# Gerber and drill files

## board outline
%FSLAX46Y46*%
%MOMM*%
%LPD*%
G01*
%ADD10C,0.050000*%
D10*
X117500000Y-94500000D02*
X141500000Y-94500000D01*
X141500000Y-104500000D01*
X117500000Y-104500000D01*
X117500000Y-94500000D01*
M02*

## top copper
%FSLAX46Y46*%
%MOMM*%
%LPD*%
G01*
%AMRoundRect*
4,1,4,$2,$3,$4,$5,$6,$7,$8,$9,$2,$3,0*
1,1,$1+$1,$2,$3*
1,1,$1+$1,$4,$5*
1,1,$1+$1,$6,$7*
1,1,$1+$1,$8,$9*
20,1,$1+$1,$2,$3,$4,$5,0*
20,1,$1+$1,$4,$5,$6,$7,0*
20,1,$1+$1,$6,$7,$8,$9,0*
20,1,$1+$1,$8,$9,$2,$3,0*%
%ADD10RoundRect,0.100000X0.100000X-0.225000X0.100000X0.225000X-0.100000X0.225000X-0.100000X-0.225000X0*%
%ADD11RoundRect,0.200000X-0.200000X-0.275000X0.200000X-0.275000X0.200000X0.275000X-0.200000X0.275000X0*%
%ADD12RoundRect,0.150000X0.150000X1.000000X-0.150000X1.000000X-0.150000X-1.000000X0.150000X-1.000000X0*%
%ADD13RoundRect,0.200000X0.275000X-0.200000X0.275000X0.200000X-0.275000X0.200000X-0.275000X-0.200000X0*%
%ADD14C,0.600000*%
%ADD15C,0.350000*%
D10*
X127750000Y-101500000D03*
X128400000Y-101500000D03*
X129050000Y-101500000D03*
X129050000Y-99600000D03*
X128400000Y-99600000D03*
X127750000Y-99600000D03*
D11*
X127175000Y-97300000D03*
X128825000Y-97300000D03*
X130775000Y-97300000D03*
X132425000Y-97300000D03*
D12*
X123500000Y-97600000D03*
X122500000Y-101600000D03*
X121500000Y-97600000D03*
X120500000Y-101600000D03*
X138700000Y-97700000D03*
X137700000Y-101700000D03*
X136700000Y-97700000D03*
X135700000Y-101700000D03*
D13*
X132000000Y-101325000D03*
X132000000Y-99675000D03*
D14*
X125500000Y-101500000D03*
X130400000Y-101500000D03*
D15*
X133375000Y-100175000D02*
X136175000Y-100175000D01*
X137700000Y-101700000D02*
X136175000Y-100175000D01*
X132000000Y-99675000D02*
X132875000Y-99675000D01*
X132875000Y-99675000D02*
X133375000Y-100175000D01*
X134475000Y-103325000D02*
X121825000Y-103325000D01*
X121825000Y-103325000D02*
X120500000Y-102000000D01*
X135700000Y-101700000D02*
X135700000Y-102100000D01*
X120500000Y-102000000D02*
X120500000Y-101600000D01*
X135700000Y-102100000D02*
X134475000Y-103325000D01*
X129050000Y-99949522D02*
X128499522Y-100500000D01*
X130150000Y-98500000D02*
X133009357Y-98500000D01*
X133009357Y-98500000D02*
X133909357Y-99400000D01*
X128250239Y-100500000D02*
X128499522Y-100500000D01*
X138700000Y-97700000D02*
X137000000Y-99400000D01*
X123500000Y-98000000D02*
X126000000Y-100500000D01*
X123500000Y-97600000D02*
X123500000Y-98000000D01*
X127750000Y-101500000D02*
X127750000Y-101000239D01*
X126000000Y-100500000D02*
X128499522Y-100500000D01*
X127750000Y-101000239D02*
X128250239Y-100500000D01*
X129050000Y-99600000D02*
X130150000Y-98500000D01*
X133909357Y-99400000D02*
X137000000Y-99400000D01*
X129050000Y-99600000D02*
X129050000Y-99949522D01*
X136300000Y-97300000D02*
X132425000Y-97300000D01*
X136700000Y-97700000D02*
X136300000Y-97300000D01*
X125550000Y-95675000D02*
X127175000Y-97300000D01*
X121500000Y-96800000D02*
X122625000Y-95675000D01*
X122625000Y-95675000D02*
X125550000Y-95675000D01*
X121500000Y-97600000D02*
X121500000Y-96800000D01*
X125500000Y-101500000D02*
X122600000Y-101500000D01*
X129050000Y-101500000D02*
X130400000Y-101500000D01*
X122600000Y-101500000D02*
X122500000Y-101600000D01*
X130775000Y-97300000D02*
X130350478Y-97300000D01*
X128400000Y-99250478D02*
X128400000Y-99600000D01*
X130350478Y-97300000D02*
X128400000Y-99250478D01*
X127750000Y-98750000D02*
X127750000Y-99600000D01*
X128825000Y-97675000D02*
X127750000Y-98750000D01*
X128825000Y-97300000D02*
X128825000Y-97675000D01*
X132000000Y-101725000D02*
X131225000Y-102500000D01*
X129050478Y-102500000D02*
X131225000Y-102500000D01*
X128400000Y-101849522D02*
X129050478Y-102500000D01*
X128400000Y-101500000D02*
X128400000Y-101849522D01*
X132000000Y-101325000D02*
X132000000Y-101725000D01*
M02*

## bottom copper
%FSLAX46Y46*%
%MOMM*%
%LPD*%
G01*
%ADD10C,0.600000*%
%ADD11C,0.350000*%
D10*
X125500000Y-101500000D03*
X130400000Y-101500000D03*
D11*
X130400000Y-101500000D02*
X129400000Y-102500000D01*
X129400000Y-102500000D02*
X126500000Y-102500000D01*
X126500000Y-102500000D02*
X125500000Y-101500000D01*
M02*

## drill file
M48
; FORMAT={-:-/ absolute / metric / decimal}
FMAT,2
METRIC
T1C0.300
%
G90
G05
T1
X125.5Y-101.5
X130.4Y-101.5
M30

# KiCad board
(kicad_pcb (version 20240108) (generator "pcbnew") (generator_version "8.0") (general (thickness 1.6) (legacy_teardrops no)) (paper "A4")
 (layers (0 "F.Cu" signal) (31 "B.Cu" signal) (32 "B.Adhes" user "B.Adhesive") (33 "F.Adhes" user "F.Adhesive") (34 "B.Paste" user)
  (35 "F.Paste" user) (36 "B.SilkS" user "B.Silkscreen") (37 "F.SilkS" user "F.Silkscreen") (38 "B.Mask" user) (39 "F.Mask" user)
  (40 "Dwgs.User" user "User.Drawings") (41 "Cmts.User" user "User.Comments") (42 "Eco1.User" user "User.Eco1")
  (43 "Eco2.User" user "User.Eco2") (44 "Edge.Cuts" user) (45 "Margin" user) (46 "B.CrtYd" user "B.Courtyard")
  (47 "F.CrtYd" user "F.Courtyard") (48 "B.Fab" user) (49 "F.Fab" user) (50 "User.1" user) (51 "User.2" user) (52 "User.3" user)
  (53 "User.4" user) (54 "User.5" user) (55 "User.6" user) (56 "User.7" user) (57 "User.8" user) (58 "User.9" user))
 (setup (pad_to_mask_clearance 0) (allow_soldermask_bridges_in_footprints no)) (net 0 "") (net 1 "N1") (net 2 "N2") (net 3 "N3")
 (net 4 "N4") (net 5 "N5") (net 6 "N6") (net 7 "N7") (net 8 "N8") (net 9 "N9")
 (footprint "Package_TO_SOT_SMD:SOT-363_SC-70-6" (layer "F.Cu") (at 128.4 100.55 90)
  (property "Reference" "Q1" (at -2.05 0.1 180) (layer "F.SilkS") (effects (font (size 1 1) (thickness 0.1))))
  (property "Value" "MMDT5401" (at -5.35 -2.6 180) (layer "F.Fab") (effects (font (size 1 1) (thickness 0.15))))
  (pad "1" smd roundrect (at -0.95 -0.65 90) (size 0.65 0.4) (layers "F.Cu" "F.Paste" "F.Mask") (roundrect_rratio 0.25) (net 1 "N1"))
  (pad "2" smd roundrect (at -0.95 0 90) (size 0.65 0.4) (layers "F.Cu" "F.Paste" "F.Mask") (roundrect_rratio 0.25) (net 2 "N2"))
  (pad "3" smd roundrect (at -0.95 0.65 90) (size 0.65 0.4) (layers "F.Cu" "F.Paste" "F.Mask") (roundrect_rratio 0.25) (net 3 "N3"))
  (pad "4" smd roundrect (at 0.95 0.65 90) (size 0.65 0.4) (layers "F.Cu" "F.Paste" "F.Mask") (roundrect_rratio 0.25) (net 1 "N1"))
  (pad "5" smd roundrect (at 0.95 0 90) (size 0.65 0.4) (layers "F.Cu" "F.Paste" "F.Mask") (roundrect_rratio 0.25) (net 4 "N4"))
  (pad "6" smd roundrect (at 0.95 -0.65 90) (size 0.65 0.4) (layers "F.Cu" "F.Paste" "F.Mask") (roundrect_rratio 0.25) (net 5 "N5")))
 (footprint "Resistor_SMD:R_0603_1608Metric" (layer "F.Cu") (at 128 97.3)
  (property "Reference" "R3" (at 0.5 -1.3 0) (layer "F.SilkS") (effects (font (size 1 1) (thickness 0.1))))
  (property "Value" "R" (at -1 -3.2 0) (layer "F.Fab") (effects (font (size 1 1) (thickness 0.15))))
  (pad "1" smd roundrect (at -0.825 0) (size 0.8 0.95) (layers "F.Cu" "F.Paste" "F.Mask") (roundrect_rratio 0.25) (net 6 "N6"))
  (pad "2" smd roundrect (at 0.825 0) (size 0.8 0.95) (layers "F.Cu" "F.Paste" "F.Mask") (roundrect_rratio 0.25) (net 5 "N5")))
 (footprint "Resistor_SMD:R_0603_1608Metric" (layer "F.Cu") (at 131.6 97.3)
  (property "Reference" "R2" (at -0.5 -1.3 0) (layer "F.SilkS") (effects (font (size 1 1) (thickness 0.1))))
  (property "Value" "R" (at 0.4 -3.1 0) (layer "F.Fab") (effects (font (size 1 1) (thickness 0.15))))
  (pad "1" smd roundrect (at -0.825 0) (size 0.8 0.95) (layers "F.Cu" "F.Paste" "F.Mask") (roundrect_rratio 0.25) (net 4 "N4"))
  (pad "2" smd roundrect (at 0.825 0) (size 0.8 0.95) (layers "F.Cu" "F.Paste" "F.Mask") (roundrect_rratio 0.25) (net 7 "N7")))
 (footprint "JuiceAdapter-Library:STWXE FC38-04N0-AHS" (layer "F.Cu") (at 122 99.6 180)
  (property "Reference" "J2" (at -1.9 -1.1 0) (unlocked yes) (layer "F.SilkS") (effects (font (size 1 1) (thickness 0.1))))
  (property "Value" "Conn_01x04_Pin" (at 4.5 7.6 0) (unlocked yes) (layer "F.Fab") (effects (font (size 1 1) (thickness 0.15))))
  (pad "1" smd roundrect (at -1.5 2 180) (size 0.6 2.3) (layers "F.Cu" "F.Paste" "F.Mask") (roundrect_rratio 0.25) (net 1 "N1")
   (thermal_bridge_angle 45))
  (pad "2" smd roundrect (at -0.5 -2 180) (size 0.6 2.3) (layers "F.Cu" "F.Paste" "F.Mask") (roundrect_rratio 0.25) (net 3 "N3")
   (thermal_bridge_angle 45))
  (pad "3" smd roundrect (at 0.5 2 180) (size 0.6 2.3) (layers "F.Cu" "F.Paste" "F.Mask") (roundrect_rratio 0.25) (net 6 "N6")
   (thermal_bridge_angle 45))
  (pad "4" smd roundrect (at 1.5 -2 180) (size 0.6 2.3) (layers "F.Cu" "F.Paste" "F.Mask") (roundrect_rratio 0.25) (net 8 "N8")
   (thermal_bridge_angle 45)))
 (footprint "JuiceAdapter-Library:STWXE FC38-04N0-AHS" (layer "F.Cu") (at 137.2 99.7 180)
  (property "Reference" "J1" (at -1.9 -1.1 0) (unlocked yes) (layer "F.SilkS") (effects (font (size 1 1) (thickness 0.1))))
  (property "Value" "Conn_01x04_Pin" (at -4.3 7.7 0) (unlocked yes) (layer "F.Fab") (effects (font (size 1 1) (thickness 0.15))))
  (pad "1" smd roundrect (at -1.5 2 180) (size 0.6 2.3) (layers "F.Cu" "F.Paste" "F.Mask") (roundrect_rratio 0.25) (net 1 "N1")
   (thermal_bridge_angle 45))
  (pad "2" smd roundrect (at -0.5 -2 180) (size 0.6 2.3) (layers "F.Cu" "F.Paste" "F.Mask") (roundrect_rratio 0.25) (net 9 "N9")
   (thermal_bridge_angle 45))
  (pad "3" smd roundrect (at 0.5 2 180) (size 0.6 2.3) (layers "F.Cu" "F.Paste" "F.Mask") (roundrect_rratio 0.25) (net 7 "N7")
   (thermal_bridge_angle 45))
  (pad "4" smd roundrect (at 1.5 -2 180) (size 0.6 2.3) (layers "F.Cu" "F.Paste" "F.Mask") (roundrect_rratio 0.25) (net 8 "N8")
   (thermal_bridge_angle 45)))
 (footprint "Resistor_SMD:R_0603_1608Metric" (layer "F.Cu") (at 132 100.5 90)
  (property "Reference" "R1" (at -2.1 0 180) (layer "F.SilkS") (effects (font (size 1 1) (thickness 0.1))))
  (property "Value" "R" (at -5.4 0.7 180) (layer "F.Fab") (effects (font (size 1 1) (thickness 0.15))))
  (pad "1" smd roundrect (at -0.825 0 90) (size 0.8 0.95) (layers "F.Cu" "F.Paste" "F.Mask") (roundrect_rratio 0.25) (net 2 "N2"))
  (pad "2" smd roundrect (at 0.825 0 90) (size 0.8 0.95) (layers "F.Cu" "F.Paste" "F.Mask") (roundrect_rratio 0.25) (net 9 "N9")))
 (gr_rect (start 117.5 94.5) (end 141.5 104.5) (stroke (width 0.05) (type default)) (fill none) (layer "Edge.Cuts"))
 (segment (start 133.375 100.175) (end 136.175 100.175) (width 0.35) (layer "F.Cu") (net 9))
 (segment (start 137.7 101.7) (end 136.175 100.175) (width 0.35) (layer "F.Cu") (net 9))
 (segment (start 132 99.675) (end 132.875 99.675) (width 0.35) (layer "F.Cu") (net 9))
 (segment (start 132.875 99.675) (end 133.375 100.175) (width 0.35) (layer "F.Cu") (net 9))
 (segment (start 134.475 103.325) (end 121.825 103.325) (width 0.35) (layer "F.Cu") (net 8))
 (segment (start 121.825 103.325) (end 120.5 102) (width 0.35) (layer "F.Cu") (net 8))
 (segment (start 135.7 101.7) (end 135.7 102.1) (width 0.35) (layer "F.Cu") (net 8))
 (segment (start 120.5 102) (end 120.5 101.6) (width 0.35) (layer "F.Cu") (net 8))
 (segment (start 135.7 102.1) (end 134.475 103.325) (width 0.35) (layer "F.Cu") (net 8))
 (segment (start 129.05 99.949522) (end 128.499522 100.5) (width 0.35) (layer "F.Cu") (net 1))
 (segment (start 130.15 98.5) (end 133.009357 98.5) (width 0.35) (layer "F.Cu") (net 1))
 (segment (start 133.009357 98.5) (end 133.909357 99.4) (width 0.35) (layer "F.Cu") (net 1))
 (segment (start 128.250239 100.5) (end 128.499522 100.5) (width 0.35) (layer "F.Cu") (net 1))
 (segment (start 138.7 97.7) (end 137 99.4) (width 0.35) (layer "F.Cu") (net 1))
 (segment (start 123.5 98) (end 126 100.5) (width 0.35) (layer "F.Cu") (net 1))
 (segment (start 123.5 97.6) (end 123.5 98) (width 0.35) (layer "F.Cu") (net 1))
 (segment (start 127.75 101.5) (end 127.75 101.000239) (width 0.35) (layer "F.Cu") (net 1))
 (segment (start 126 100.5) (end 128.499522 100.5) (width 0.35) (layer "F.Cu") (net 1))
 (segment (start 127.75 101.000239) (end 128.250239 100.5) (width 0.35) (layer "F.Cu") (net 1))
 (segment (start 129.05 99.6) (end 130.15 98.5) (width 0.35) (layer "F.Cu") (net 1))
 (segment (start 133.909357 99.4) (end 137 99.4) (width 0.35) (layer "F.Cu") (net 1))
 (segment (start 129.05 99.6) (end 129.05 99.949522) (width 0.35) (layer "F.Cu") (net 1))
 (segment (start 136.3 97.3) (end 132.425 97.3) (width 0.35) (layer "F.Cu") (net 7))
 (segment (start 136.7 97.7) (end 136.3 97.3) (width 0.35) (layer "F.Cu") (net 7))
 (segment (start 125.55 95.675) (end 127.175 97.3) (width 0.35) (layer "F.Cu") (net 6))
 (segment (start 121.5 96.8) (end 122.625 95.675) (width 0.35) (layer "F.Cu") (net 6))
 (segment (start 122.625 95.675) (end 125.55 95.675) (width 0.35) (layer "F.Cu") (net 6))
 (segment (start 121.5 97.6) (end 121.5 96.8) (width 0.35) (layer "F.Cu") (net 6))
 (segment (start 125.5 101.5) (end 122.6 101.5) (width 0.35) (layer "F.Cu") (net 3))
 (segment (start 129.05 101.5) (end 130.4 101.5) (width 0.35) (layer "F.Cu") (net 3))
 (segment (start 122.6 101.5) (end 122.5 101.6) (width 0.35) (layer "F.Cu") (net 3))
 (via (at 125.5 101.5) (size 0.6) (drill 0.3) (layers "F.Cu" "B.Cu") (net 3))
 (via (at 130.4 101.5) (size 0.6) (drill 0.3) (layers "F.Cu" "B.Cu") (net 3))
 (segment (start 130.4 101.5) (end 129.4 102.5) (width 0.35) (layer "B.Cu") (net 3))
 (segment (start 129.4 102.5) (end 126.5 102.5) (width 0.35) (layer "B.Cu") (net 3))
 (segment (start 126.5 102.5) (end 125.5 101.5) (width 0.35) (layer "B.Cu") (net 3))
 (segment (start 130.775 97.3) (end 130.350478 97.3) (width 0.35) (layer "F.Cu") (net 4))
 (segment (start 128.4 99.250478) (end 128.4 99.6) (width 0.35) (layer "F.Cu") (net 4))
 (segment (start 130.350478 97.3) (end 128.4 99.250478) (width 0.35) (layer "F.Cu") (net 4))
 (segment (start 127.75 98.75) (end 127.75 99.6) (width 0.35) (layer "F.Cu") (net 5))
 (segment (start 128.825 97.675) (end 127.75 98.75) (width 0.35) (layer "F.Cu") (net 5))
 (segment (start 128.825 97.3) (end 128.825 97.675) (width 0.35) (layer "F.Cu") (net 5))
 (segment (start 132 101.725) (end 131.225 102.5) (width 0.35) (layer "F.Cu") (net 2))
 (segment (start 129.050478 102.5) (end 131.225 102.5) (width 0.35) (layer "F.Cu") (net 2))
 (segment (start 128.4 101.849522) (end 129.050478 102.5) (width 0.35) (layer "F.Cu") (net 2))
 (segment (start 128.4 101.5) (end 128.4 101.849522) (width 0.35) (layer "F.Cu") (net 2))
 (segment (start 132 101.325) (end 132 101.725) (width 0.35) (layer "F.Cu") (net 2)))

